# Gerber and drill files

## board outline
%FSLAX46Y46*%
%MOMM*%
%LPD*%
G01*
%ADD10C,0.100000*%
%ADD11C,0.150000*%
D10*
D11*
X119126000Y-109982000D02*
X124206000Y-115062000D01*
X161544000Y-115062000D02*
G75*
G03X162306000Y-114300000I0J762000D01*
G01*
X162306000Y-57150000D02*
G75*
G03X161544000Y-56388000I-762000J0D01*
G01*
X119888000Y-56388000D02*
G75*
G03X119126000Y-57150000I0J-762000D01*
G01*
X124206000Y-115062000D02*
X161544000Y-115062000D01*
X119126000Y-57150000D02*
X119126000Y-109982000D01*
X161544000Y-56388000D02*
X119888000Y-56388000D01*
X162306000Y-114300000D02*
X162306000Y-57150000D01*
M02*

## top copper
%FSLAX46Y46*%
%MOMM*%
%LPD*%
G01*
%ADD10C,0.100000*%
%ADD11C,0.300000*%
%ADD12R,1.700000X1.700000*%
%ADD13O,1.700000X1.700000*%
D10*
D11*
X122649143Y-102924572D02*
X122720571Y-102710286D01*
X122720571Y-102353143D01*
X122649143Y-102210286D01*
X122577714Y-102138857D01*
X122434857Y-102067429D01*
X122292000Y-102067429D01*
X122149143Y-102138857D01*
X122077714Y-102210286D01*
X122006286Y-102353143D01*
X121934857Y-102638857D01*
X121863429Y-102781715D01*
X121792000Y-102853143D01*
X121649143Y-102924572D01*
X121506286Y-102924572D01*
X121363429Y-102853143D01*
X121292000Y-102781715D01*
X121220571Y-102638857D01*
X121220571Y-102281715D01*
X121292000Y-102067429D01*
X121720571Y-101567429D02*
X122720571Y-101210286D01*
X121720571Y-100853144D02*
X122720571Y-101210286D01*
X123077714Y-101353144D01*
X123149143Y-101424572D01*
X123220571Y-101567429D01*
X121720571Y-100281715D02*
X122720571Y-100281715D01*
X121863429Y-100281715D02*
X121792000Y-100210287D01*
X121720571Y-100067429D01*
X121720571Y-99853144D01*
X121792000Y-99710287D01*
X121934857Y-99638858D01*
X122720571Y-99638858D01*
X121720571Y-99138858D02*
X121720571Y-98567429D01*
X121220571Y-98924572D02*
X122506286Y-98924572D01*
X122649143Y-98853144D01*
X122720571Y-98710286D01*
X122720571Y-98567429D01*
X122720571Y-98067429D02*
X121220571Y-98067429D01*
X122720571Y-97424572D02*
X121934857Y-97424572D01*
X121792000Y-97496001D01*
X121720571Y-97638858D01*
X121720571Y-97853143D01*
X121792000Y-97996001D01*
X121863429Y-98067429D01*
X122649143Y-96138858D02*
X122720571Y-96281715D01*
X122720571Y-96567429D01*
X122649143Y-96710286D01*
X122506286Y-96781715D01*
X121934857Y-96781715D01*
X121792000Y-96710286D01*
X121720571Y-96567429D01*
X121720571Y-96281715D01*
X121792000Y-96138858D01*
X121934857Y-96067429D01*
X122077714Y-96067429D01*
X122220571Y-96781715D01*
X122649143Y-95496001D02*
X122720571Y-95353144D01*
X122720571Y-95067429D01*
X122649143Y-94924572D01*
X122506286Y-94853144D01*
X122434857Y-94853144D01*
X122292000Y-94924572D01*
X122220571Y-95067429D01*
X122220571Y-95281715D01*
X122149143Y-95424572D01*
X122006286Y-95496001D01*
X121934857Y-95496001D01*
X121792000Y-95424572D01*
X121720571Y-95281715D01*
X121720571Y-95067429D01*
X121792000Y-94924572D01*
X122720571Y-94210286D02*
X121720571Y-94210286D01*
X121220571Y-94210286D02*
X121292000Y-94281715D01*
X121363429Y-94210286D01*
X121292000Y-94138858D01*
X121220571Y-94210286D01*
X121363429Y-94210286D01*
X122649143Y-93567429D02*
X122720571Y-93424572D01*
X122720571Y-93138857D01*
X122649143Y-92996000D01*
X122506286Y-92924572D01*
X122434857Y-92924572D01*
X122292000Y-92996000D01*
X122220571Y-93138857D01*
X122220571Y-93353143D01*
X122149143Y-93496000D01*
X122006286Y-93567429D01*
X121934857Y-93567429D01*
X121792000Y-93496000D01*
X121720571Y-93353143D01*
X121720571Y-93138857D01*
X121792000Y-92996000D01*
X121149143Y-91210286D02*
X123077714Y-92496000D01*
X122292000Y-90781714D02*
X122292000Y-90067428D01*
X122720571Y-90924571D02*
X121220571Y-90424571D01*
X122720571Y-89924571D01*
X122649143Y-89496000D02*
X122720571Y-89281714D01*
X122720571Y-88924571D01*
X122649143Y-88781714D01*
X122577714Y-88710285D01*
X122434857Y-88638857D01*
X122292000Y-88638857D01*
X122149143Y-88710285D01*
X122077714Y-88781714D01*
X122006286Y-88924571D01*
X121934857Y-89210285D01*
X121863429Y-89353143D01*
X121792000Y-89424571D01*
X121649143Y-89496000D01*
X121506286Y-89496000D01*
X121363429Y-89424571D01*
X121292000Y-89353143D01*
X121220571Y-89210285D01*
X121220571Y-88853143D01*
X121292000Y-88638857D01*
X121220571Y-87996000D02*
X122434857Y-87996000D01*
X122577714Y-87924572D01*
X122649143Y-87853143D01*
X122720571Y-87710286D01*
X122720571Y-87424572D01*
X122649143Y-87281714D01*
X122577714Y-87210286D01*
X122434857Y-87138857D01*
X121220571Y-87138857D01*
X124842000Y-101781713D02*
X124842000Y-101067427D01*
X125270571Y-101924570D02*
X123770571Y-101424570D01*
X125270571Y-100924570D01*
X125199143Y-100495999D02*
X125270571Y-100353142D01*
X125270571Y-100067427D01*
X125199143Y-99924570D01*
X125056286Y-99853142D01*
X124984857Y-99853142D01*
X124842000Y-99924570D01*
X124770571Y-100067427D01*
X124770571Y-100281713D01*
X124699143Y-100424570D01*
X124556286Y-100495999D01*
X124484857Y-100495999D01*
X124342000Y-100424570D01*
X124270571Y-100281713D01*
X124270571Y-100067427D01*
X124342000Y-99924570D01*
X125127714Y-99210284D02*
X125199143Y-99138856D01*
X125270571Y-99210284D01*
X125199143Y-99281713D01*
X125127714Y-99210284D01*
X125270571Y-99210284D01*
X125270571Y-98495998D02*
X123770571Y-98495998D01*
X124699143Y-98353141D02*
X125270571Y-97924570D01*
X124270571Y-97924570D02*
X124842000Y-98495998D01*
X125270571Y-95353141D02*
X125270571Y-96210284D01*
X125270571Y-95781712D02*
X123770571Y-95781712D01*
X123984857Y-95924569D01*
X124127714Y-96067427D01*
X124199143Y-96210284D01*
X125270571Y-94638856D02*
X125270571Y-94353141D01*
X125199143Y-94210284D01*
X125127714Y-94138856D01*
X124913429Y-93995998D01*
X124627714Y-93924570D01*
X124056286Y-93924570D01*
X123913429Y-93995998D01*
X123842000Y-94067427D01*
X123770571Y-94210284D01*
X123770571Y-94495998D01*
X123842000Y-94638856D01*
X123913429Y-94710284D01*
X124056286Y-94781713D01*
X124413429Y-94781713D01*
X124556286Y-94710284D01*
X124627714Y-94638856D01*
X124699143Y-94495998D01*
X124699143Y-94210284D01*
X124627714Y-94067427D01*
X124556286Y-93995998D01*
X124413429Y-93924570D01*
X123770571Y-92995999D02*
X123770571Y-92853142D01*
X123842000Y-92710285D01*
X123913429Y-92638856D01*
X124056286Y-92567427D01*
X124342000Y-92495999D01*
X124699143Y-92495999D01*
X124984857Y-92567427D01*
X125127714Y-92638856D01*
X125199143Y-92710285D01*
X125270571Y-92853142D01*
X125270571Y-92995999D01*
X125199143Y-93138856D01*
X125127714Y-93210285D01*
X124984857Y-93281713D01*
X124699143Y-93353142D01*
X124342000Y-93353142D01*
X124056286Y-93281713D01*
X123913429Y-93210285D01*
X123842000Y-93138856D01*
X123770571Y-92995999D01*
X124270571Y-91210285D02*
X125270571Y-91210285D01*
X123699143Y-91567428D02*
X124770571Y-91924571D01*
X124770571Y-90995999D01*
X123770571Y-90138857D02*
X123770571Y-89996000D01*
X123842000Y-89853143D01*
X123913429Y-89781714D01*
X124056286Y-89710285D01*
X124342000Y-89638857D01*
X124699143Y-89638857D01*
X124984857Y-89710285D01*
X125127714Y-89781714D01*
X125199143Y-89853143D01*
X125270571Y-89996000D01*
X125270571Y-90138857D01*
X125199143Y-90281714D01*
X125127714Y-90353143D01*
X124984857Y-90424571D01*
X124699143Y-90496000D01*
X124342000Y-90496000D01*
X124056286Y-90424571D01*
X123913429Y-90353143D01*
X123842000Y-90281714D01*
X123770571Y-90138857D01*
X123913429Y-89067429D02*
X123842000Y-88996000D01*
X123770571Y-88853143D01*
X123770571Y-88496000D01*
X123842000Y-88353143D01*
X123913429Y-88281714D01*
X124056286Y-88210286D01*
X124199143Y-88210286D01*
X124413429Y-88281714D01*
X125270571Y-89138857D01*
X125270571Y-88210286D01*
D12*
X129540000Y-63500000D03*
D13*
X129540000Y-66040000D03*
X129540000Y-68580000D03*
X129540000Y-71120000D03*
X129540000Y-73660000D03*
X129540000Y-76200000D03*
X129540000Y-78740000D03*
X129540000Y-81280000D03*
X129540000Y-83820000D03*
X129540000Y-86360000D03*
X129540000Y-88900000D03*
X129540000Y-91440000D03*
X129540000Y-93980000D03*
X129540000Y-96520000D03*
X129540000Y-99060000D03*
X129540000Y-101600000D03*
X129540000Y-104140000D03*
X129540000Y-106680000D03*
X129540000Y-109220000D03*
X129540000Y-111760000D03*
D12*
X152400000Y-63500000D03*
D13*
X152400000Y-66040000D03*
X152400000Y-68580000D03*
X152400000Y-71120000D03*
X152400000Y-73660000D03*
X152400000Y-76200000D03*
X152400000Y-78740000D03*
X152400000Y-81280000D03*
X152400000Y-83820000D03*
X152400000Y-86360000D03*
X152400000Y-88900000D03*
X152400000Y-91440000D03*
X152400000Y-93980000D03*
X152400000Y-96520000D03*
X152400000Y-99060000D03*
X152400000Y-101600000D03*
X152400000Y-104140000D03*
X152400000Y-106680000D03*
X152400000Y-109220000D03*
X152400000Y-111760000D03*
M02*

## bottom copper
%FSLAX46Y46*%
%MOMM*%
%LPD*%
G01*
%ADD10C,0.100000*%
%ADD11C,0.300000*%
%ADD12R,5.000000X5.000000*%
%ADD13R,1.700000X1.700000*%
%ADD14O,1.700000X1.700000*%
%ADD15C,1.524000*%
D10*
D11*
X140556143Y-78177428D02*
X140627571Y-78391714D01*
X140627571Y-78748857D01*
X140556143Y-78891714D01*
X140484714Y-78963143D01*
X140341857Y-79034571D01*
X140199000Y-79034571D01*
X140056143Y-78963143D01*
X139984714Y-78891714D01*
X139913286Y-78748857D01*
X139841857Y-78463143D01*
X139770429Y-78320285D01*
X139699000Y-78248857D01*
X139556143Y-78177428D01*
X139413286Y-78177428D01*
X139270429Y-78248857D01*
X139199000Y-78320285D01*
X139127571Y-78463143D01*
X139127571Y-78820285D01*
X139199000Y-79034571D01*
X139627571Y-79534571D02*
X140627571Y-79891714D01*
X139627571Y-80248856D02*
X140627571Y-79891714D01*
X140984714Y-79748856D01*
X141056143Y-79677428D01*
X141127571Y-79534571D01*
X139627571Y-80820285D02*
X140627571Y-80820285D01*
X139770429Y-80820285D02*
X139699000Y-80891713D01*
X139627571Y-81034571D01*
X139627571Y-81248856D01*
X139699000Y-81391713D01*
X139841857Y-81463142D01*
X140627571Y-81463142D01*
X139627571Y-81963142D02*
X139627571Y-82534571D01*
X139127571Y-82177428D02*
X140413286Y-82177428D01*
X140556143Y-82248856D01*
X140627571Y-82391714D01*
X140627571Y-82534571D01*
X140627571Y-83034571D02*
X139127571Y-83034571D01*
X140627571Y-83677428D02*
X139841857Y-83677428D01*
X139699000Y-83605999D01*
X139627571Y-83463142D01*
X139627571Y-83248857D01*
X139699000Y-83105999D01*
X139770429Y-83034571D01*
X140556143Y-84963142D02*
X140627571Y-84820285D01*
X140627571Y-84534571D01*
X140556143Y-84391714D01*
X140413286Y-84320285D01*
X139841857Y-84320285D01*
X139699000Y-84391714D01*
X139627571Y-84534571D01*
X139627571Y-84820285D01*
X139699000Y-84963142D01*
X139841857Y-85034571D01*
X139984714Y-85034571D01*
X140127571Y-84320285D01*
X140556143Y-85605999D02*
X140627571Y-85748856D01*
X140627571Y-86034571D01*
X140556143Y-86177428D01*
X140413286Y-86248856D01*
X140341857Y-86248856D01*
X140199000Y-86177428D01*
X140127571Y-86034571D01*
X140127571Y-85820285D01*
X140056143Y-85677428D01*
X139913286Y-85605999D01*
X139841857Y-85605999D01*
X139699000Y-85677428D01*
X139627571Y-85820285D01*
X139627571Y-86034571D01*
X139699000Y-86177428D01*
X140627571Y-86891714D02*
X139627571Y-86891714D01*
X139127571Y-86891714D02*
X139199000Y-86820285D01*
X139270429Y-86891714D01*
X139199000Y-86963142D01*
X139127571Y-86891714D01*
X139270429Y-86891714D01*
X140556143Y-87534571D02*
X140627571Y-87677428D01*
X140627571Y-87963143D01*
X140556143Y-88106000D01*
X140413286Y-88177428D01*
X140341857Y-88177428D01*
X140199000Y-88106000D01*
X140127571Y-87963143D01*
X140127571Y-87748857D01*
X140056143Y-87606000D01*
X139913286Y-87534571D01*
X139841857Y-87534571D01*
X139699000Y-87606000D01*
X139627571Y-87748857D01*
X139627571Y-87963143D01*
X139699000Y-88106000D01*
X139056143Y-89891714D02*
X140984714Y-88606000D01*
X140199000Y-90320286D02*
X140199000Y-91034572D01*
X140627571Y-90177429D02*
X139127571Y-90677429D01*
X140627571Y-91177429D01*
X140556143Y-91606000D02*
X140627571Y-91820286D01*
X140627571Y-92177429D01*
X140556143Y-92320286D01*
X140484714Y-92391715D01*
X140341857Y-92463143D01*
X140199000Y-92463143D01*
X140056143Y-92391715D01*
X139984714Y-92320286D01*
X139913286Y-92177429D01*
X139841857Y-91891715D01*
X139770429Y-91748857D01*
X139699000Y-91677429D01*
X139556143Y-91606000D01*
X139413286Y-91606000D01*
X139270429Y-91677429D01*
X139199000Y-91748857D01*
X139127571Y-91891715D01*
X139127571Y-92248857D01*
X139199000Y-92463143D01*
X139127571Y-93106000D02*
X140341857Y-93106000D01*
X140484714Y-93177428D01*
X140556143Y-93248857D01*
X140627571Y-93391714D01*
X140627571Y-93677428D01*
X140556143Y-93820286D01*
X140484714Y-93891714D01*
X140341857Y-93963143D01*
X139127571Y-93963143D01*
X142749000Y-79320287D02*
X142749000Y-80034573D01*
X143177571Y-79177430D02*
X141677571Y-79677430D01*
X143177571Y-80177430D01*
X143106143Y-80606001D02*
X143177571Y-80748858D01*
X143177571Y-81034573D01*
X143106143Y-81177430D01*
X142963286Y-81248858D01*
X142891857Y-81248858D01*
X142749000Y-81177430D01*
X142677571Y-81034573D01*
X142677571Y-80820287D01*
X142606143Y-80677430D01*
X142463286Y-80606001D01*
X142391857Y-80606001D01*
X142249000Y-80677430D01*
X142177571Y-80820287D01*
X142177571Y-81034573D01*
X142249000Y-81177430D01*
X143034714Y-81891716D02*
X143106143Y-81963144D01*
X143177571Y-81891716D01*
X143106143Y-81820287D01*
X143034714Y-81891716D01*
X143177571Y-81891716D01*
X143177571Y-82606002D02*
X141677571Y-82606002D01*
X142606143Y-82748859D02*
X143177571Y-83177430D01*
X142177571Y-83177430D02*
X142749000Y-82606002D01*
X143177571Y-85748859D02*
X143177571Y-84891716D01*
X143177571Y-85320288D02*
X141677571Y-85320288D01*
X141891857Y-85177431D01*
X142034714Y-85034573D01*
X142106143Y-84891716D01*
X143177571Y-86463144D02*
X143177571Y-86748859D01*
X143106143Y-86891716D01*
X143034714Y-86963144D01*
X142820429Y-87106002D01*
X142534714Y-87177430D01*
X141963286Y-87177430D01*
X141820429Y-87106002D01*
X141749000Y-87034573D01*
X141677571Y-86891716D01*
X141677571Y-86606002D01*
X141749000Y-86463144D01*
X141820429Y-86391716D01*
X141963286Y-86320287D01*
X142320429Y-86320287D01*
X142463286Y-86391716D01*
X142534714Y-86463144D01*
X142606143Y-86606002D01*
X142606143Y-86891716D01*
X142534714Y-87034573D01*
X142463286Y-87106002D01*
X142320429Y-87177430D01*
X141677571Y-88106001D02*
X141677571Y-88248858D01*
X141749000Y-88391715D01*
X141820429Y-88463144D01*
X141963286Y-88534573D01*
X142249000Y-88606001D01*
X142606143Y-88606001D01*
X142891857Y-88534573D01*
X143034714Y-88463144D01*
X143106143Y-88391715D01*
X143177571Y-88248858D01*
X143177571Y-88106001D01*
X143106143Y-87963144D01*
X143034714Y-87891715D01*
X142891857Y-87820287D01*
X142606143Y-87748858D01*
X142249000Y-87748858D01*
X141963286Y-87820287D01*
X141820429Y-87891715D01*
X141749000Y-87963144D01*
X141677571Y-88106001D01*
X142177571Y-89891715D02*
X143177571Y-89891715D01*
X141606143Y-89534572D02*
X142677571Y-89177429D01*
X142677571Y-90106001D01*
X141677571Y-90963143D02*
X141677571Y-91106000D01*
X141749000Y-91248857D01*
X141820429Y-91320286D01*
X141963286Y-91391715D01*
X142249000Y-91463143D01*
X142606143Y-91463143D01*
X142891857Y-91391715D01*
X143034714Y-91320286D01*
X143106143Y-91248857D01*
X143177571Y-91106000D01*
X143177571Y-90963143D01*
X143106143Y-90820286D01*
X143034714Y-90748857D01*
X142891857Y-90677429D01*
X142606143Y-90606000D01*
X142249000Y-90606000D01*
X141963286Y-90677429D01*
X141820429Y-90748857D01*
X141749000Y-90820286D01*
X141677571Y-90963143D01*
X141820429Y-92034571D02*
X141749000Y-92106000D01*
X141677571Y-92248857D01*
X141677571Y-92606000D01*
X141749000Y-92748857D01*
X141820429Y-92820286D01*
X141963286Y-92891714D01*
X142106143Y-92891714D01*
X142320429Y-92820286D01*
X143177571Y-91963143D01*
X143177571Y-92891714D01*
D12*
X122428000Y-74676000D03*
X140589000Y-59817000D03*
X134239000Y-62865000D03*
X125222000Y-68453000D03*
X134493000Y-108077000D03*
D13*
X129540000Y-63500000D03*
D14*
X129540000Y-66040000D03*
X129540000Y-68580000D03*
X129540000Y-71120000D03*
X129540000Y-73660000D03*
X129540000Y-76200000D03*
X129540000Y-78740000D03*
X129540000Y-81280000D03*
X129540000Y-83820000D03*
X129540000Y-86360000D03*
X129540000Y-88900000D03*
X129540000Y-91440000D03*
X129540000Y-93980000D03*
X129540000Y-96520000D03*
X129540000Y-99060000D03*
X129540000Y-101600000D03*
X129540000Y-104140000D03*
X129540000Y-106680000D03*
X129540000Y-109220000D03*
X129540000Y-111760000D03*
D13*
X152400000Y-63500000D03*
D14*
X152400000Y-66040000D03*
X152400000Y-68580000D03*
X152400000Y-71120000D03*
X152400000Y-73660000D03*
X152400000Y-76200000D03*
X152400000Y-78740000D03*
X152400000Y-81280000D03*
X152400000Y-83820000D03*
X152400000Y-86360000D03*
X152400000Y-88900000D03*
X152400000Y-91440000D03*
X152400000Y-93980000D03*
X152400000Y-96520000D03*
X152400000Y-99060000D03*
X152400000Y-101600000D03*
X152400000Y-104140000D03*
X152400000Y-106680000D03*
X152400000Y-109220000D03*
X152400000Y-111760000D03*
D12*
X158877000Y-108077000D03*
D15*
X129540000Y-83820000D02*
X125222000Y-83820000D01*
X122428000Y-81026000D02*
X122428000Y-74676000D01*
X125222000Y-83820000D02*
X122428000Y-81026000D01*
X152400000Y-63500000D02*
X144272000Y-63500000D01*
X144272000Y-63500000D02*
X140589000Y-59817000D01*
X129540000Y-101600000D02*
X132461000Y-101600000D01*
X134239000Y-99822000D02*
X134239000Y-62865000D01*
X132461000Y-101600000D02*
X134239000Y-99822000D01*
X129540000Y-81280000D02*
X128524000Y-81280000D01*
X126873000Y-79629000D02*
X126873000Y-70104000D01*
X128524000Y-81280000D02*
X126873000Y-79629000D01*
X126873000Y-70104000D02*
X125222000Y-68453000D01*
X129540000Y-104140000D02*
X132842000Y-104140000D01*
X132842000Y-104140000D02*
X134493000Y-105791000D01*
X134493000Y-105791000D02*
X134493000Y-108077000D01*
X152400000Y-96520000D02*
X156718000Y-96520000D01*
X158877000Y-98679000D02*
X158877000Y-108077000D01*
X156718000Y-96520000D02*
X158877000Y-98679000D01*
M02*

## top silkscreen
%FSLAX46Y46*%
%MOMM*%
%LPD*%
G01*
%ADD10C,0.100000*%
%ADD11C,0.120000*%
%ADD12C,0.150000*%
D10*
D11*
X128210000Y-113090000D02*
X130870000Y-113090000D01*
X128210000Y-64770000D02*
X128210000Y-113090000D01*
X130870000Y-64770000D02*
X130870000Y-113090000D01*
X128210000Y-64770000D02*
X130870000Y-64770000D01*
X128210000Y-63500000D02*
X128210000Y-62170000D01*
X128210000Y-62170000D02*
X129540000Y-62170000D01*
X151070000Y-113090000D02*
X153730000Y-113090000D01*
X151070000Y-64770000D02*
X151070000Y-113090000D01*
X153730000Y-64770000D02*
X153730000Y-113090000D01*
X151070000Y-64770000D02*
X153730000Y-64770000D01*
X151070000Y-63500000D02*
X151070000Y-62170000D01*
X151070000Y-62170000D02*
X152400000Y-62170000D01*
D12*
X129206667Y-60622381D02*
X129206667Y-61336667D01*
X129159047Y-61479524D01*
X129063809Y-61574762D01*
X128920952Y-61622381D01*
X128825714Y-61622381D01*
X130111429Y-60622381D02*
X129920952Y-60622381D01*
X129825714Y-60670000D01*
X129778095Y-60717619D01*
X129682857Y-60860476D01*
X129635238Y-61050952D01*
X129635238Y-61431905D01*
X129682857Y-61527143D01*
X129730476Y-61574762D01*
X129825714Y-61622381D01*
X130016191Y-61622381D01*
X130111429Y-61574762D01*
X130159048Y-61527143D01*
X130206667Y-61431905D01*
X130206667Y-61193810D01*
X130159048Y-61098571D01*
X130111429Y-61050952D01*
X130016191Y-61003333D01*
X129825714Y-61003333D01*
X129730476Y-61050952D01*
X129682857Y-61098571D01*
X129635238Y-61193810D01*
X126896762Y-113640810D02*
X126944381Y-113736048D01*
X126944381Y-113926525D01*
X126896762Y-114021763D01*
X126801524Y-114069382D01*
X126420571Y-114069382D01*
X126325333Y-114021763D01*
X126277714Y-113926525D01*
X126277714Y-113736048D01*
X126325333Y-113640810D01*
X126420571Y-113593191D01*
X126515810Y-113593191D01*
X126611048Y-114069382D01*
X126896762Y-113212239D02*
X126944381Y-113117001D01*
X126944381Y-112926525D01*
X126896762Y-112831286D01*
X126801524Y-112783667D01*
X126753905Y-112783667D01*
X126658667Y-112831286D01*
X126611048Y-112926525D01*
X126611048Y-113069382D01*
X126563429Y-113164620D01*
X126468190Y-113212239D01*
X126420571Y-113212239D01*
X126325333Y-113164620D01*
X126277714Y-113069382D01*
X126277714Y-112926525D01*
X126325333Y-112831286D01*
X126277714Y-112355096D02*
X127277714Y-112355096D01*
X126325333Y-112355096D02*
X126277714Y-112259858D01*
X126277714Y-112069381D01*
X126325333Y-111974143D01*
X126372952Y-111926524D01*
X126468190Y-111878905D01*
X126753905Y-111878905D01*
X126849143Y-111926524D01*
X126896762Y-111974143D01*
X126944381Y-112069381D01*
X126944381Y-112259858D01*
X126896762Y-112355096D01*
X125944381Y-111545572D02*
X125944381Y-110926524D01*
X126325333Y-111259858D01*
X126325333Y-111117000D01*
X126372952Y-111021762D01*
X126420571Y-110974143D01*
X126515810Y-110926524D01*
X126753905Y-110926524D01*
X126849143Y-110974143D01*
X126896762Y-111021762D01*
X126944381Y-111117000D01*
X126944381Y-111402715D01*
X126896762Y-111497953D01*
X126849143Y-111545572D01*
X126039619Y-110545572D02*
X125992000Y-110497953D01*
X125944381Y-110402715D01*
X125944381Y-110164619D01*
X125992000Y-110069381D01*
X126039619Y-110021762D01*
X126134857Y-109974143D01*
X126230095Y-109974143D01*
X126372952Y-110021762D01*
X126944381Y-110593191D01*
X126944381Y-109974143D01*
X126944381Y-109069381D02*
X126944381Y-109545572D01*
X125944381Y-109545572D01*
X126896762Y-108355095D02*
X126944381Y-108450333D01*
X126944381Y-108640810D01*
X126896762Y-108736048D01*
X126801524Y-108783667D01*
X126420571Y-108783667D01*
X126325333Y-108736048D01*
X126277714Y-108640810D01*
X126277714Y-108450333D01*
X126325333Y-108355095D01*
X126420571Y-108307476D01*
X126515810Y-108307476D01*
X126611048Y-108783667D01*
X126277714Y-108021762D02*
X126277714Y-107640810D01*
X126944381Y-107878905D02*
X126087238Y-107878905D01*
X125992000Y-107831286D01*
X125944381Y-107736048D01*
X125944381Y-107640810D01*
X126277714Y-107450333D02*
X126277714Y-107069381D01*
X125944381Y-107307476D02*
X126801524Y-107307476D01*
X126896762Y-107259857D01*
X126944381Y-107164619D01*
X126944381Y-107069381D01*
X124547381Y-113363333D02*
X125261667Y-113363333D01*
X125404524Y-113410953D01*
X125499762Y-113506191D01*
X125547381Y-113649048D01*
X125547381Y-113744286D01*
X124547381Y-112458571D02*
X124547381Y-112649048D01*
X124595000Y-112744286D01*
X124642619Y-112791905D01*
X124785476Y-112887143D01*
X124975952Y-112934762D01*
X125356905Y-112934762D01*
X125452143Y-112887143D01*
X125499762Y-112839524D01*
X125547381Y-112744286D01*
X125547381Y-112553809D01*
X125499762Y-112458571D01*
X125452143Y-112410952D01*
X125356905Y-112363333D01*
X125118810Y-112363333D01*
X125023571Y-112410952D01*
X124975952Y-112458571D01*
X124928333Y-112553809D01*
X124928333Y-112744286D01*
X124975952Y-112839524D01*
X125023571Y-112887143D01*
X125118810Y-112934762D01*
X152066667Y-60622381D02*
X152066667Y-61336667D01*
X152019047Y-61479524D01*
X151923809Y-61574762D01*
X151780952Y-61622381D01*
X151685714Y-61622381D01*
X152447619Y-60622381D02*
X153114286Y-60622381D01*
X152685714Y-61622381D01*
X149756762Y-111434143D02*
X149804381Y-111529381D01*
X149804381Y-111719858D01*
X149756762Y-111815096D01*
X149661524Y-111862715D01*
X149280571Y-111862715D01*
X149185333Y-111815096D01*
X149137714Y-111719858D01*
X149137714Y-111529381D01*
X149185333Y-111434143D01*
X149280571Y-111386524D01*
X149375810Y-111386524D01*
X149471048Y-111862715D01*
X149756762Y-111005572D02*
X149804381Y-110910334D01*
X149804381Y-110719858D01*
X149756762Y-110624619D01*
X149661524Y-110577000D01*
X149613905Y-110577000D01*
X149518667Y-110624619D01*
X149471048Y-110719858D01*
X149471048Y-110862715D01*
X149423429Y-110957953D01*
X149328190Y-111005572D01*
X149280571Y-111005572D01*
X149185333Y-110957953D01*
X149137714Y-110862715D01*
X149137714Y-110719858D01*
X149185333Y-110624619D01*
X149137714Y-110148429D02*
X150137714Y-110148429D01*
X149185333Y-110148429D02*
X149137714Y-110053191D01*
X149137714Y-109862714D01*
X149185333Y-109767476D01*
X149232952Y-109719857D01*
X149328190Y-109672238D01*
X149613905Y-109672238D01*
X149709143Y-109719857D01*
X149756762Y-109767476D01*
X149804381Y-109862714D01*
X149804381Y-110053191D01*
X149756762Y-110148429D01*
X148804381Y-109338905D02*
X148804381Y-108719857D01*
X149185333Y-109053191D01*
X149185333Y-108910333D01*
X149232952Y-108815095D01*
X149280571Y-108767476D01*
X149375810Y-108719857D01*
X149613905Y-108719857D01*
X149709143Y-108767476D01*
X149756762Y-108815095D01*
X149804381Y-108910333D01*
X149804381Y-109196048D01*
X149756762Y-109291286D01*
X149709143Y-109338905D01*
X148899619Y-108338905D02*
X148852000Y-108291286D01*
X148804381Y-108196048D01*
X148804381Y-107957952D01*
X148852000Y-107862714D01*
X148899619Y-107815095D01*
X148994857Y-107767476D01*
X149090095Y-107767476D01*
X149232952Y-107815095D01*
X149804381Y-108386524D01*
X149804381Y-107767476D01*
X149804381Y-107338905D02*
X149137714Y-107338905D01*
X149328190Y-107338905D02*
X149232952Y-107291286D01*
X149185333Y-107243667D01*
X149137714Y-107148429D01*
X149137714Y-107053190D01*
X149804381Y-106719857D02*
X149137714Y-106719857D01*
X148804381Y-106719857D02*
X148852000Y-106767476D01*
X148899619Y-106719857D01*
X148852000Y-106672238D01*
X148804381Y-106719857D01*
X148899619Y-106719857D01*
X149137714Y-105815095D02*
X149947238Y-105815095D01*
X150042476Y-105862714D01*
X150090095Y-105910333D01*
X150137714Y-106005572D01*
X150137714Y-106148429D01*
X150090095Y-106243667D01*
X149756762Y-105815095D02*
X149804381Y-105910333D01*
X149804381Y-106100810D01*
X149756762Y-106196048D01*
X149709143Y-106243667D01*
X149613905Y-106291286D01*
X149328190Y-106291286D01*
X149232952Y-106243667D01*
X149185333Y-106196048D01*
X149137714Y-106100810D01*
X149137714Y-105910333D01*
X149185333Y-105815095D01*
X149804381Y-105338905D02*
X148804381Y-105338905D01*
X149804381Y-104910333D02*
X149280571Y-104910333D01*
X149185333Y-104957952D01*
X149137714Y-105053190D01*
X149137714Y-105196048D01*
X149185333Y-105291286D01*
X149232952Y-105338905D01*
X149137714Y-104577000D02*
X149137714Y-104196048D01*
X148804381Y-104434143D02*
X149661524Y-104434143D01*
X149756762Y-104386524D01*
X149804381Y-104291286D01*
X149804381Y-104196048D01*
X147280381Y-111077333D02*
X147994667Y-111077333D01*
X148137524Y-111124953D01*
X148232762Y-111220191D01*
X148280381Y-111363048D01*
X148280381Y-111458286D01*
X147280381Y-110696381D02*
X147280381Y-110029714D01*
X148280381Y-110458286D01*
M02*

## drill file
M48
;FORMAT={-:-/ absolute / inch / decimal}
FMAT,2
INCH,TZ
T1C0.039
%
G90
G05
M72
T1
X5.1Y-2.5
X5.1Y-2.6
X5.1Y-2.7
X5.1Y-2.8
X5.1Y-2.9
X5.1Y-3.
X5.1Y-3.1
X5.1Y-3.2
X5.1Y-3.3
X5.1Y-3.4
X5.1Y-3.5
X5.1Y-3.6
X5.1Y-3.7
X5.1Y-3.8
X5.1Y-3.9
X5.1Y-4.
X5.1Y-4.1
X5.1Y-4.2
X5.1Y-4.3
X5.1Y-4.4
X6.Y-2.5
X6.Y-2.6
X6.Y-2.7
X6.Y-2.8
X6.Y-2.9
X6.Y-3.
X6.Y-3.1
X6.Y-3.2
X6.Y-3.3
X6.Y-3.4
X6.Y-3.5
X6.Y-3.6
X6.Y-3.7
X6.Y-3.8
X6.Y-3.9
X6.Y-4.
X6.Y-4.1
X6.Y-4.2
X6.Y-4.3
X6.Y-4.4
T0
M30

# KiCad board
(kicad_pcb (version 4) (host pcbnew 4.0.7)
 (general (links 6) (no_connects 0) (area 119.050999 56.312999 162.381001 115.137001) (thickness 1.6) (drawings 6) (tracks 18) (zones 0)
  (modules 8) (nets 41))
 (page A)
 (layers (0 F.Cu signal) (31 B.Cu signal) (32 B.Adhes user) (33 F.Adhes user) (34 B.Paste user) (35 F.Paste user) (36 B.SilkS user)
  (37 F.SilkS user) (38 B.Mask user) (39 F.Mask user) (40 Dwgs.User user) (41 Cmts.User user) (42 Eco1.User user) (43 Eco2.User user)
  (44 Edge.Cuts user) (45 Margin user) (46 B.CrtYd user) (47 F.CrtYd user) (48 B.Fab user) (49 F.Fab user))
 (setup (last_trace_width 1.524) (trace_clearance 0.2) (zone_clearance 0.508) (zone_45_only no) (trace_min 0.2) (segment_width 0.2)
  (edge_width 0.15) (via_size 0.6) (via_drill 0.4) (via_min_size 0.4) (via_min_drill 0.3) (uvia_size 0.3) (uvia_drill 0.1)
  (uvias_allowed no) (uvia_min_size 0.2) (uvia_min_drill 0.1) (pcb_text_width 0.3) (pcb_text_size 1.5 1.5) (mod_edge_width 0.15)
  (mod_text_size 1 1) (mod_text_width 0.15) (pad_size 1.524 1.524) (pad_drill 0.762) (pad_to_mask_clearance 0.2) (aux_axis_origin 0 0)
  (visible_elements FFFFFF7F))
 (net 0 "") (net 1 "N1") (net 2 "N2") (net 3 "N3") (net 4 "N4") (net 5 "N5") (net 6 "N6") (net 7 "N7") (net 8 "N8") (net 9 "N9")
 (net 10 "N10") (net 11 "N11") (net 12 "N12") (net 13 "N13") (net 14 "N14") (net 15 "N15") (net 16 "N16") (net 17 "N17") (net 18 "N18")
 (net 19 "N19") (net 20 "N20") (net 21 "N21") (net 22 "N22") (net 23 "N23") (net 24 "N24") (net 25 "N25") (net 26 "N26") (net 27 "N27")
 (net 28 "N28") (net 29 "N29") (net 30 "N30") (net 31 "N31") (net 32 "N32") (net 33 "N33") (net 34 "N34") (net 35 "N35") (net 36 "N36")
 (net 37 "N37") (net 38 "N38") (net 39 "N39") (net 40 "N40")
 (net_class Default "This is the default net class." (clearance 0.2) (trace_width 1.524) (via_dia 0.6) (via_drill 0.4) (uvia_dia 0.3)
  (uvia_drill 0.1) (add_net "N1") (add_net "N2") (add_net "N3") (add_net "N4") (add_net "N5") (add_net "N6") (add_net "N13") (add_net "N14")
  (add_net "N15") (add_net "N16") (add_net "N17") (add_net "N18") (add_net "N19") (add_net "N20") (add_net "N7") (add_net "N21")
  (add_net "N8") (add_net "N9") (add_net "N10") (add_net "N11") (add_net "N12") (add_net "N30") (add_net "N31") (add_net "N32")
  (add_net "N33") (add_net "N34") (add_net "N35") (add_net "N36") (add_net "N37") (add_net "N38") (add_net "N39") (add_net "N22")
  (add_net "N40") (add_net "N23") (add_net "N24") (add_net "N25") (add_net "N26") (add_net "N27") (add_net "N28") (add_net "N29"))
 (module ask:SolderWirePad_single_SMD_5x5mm (layer B.Cu) (at 122.428 74.676)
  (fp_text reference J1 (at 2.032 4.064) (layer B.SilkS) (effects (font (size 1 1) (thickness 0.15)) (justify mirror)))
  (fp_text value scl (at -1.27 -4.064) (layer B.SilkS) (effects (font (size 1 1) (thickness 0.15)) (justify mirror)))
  (pad 1 smd rect (at 0 0) (size 5 5) (layers B.Cu B.Paste B.Mask) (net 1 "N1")))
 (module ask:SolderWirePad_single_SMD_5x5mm (layer B.Cu) (at 140.589 59.817)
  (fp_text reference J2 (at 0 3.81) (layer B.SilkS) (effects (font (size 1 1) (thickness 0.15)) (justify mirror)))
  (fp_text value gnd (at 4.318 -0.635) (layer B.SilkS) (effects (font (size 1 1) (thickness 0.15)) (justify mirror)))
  (pad 1 smd rect (at 0 0) (size 5 5) (layers B.Cu B.Paste B.Mask) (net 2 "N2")))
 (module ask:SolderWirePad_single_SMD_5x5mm (layer B.Cu) (at 134.239 62.865)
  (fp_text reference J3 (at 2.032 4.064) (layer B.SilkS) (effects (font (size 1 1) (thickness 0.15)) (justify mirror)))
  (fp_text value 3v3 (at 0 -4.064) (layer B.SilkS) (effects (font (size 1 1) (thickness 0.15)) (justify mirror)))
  (pad 1 smd rect (at 0 0) (size 5 5) (layers B.Cu B.Paste B.Mask) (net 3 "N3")))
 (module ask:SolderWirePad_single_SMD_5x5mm (layer B.Cu) (at 125.222 68.453)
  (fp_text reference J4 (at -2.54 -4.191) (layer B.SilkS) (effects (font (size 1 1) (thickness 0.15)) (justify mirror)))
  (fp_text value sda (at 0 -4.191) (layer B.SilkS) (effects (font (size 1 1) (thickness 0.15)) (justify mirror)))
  (pad 1 smd rect (at 0 0) (size 5 5) (layers B.Cu B.Paste B.Mask) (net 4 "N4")))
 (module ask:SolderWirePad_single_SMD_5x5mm (layer B.Cu) (at 134.493 108.077)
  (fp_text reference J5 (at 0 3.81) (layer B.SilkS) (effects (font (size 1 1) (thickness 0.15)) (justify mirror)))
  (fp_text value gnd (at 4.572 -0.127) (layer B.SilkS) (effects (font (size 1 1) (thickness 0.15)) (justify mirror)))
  (pad 1 smd rect (at 0 0) (size 5 5) (layers B.Cu B.Paste B.Mask) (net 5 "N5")))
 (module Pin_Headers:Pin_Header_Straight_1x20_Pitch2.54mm (layer F.Cu) (at 129.54 63.5)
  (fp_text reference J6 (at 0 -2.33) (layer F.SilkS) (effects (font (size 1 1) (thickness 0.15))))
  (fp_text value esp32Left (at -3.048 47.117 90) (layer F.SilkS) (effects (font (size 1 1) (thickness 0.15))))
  (fp_line (start -1.33 49.59) (end 1.33 49.59) (layer F.SilkS) (width 0.12))
  (fp_line (start -1.33 1.27) (end -1.33 49.59) (layer F.SilkS) (width 0.12))
  (fp_line (start 1.33 1.27) (end 1.33 49.59) (layer F.SilkS) (width 0.12))
  (fp_line (start -1.33 1.27) (end 1.33 1.27) (layer F.SilkS) (width 0.12))
  (fp_line (start -1.33 0) (end -1.33 -1.33) (layer F.SilkS) (width 0.12))
  (fp_line (start -1.33 -1.33) (end 0 -1.33) (layer F.SilkS) (width 0.12))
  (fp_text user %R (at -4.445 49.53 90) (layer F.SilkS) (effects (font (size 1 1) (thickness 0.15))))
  (pad 1 thru_hole rect (at 0 0) (size 1.7 1.7) (drill 1) (layers *.Cu *.Mask) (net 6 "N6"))
  (pad 2 thru_hole oval (at 0 2.54) (size 1.7 1.7) (drill 1) (layers *.Cu *.Mask) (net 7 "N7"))
  (pad 3 thru_hole oval (at 0 5.08) (size 1.7 1.7) (drill 1) (layers *.Cu *.Mask) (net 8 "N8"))
  (pad 4 thru_hole oval (at 0 7.62) (size 1.7 1.7) (drill 1) (layers *.Cu *.Mask) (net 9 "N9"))
  (pad 5 thru_hole oval (at 0 10.16) (size 1.7 1.7) (drill 1) (layers *.Cu *.Mask) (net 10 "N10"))
  (pad 6 thru_hole oval (at 0 12.7) (size 1.7 1.7) (drill 1) (layers *.Cu *.Mask) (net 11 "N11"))
  (pad 7 thru_hole oval (at 0 15.24) (size 1.7 1.7) (drill 1) (layers *.Cu *.Mask) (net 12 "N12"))
  (pad 8 thru_hole oval (at 0 17.78) (size 1.7 1.7) (drill 1) (layers *.Cu *.Mask) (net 4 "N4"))
  (pad 9 thru_hole oval (at 0 20.32) (size 1.7 1.7) (drill 1) (layers *.Cu *.Mask) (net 1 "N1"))
  (pad 10 thru_hole oval (at 0 22.86) (size 1.7 1.7) (drill 1) (layers *.Cu *.Mask) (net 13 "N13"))
  (pad 11 thru_hole oval (at 0 25.4) (size 1.7 1.7) (drill 1) (layers *.Cu *.Mask) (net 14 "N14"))
  (pad 12 thru_hole oval (at 0 27.94) (size 1.7 1.7) (drill 1) (layers *.Cu *.Mask) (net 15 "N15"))
  (pad 13 thru_hole oval (at 0 30.48) (size 1.7 1.7) (drill 1) (layers *.Cu *.Mask) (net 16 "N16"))
  (pad 14 thru_hole oval (at 0 33.02) (size 1.7 1.7) (drill 1) (layers *.Cu *.Mask) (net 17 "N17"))
  (pad 15 thru_hole oval (at 0 35.56) (size 1.7 1.7) (drill 1) (layers *.Cu *.Mask) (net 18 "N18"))
  (pad 16 thru_hole oval (at 0 38.1) (size 1.7 1.7) (drill 1) (layers *.Cu *.Mask) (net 3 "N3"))
  (pad 17 thru_hole oval (at 0 40.64) (size 1.7 1.7) (drill 1) (layers *.Cu *.Mask) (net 5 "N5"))
  (pad 18 thru_hole oval (at 0 43.18) (size 1.7 1.7) (drill 1) (layers *.Cu *.Mask) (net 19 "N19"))
  (pad 19 thru_hole oval (at 0 45.72) (size 1.7 1.7) (drill 1) (layers *.Cu *.Mask) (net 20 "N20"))
  (pad 20 thru_hole oval (at 0 48.26) (size 1.7 1.7) (drill 1) (layers *.Cu *.Mask) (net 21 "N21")))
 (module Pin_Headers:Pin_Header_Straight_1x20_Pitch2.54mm (layer F.Cu) (at 152.4 63.5)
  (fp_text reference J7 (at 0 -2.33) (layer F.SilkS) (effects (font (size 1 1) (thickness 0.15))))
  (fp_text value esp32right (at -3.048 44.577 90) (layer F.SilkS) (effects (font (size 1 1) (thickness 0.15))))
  (fp_line (start -1.33 49.59) (end 1.33 49.59) (layer F.SilkS) (width 0.12))
  (fp_line (start -1.33 1.27) (end -1.33 49.59) (layer F.SilkS) (width 0.12))
  (fp_line (start 1.33 1.27) (end 1.33 49.59) (layer F.SilkS) (width 0.12))
  (fp_line (start -1.33 1.27) (end 1.33 1.27) (layer F.SilkS) (width 0.12))
  (fp_line (start -1.33 0) (end -1.33 -1.33) (layer F.SilkS) (width 0.12))
  (fp_line (start -1.33 -1.33) (end 0 -1.33) (layer F.SilkS) (width 0.12))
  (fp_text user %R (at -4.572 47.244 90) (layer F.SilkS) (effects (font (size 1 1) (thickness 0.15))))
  (pad 1 thru_hole rect (at 0 0) (size 1.7 1.7) (drill 1) (layers *.Cu *.Mask) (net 2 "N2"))
  (pad 2 thru_hole oval (at 0 2.54) (size 1.7 1.7) (drill 1) (layers *.Cu *.Mask) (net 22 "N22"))
  (pad 3 thru_hole oval (at 0 5.08) (size 1.7 1.7) (drill 1) (layers *.Cu *.Mask) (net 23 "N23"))
  (pad 4 thru_hole oval (at 0 7.62) (size 1.7 1.7) (drill 1) (layers *.Cu *.Mask) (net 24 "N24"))
  (pad 5 thru_hole oval (at 0 10.16) (size 1.7 1.7) (drill 1) (layers *.Cu *.Mask) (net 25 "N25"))
  (pad 6 thru_hole oval (at 0 12.7) (size 1.7 1.7) (drill 1) (layers *.Cu *.Mask) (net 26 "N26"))
  (pad 7 thru_hole oval (at 0 15.24) (size 1.7 1.7) (drill 1) (layers *.Cu *.Mask) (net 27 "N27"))
  (pad 8 thru_hole oval (at 0 17.78) (size 1.7 1.7) (drill 1) (layers *.Cu *.Mask) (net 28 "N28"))
  (pad 9 thru_hole oval (at 0 20.32) (size 1.7 1.7) (drill 1) (layers *.Cu *.Mask) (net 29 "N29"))
  (pad 10 thru_hole oval (at 0 22.86) (size 1.7 1.7) (drill 1) (layers *.Cu *.Mask) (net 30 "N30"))
  (pad 11 thru_hole oval (at 0 25.4) (size 1.7 1.7) (drill 1) (layers *.Cu *.Mask) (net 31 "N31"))
  (pad 12 thru_hole oval (at 0 27.94) (size 1.7 1.7) (drill 1) (layers *.Cu *.Mask) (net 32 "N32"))
  (pad 13 thru_hole oval (at 0 30.48) (size 1.7 1.7) (drill 1) (layers *.Cu *.Mask) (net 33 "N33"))
  (pad 14 thru_hole oval (at 0 33.02) (size 1.7 1.7) (drill 1) (layers *.Cu *.Mask) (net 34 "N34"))
  (pad 15 thru_hole oval (at 0 35.56) (size 1.7 1.7) (drill 1) (layers *.Cu *.Mask) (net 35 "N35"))
  (pad 16 thru_hole oval (at 0 38.1) (size 1.7 1.7) (drill 1) (layers *.Cu *.Mask) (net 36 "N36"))
  (pad 17 thru_hole oval (at 0 40.64) (size 1.7 1.7) (drill 1) (layers *.Cu *.Mask) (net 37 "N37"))
  (pad 18 thru_hole oval (at 0 43.18) (size 1.7 1.7) (drill 1) (layers *.Cu *.Mask) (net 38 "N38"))
  (pad 19 thru_hole oval (at 0 45.72) (size 1.7 1.7) (drill 1) (layers *.Cu *.Mask) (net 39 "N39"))
  (pad 20 thru_hole oval (at 0 48.26) (size 1.7 1.7) (drill 1) (layers *.Cu *.Mask) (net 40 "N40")))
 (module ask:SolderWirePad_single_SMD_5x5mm (layer B.Cu) (at 158.877 108.077)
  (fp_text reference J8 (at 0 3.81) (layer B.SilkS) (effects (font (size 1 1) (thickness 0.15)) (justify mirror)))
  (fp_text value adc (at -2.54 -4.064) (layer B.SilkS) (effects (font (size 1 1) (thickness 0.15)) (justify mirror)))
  (pad 1 smd rect (at 0 0) (size 5 5) (layers B.Cu B.Paste B.Mask) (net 34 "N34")))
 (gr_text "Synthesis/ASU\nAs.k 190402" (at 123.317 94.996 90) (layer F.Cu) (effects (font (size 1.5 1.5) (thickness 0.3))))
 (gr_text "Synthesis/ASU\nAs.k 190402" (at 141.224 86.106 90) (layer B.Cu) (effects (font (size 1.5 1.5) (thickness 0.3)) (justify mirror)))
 (gr_line (start 119.126 115.062) (end 162.306 115.062) (angle 90) (layer Edge.Cuts) (width 0.15))
 (gr_line (start 119.126 56.388) (end 119.126 115.062) (angle 90) (layer Edge.Cuts) (width 0.15))
 (gr_line (start 162.306 56.388) (end 119.126 56.388) (angle 90) (layer Edge.Cuts) (width 0.15))
 (gr_line (start 162.306 115.062) (end 162.306 56.388) (angle 90) (layer Edge.Cuts) (width 0.15))
 (segment (start 129.54 83.82) (end 125.222 83.82) (width 1.524) (layer B.Cu) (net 1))
 (segment (start 122.428 81.026) (end 122.428 74.676) (width 1.524) (layer B.Cu) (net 1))
 (segment (start 125.222 83.82) (end 122.428 81.026) (width 1.524) (layer B.Cu) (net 1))
 (segment (start 152.4 63.5) (end 144.272 63.5) (width 1.524) (layer B.Cu) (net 2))
 (segment (start 144.272 63.5) (end 140.589 59.817) (width 1.524) (layer B.Cu) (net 2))
 (segment (start 129.54 101.6) (end 132.461 101.6) (width 1.524) (layer B.Cu) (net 3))
 (segment (start 134.239 99.822) (end 134.239 62.865) (width 1.524) (layer B.Cu) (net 3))
 (segment (start 132.461 101.6) (end 134.239 99.822) (width 1.524) (layer B.Cu) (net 3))
 (segment (start 129.54 81.28) (end 128.524 81.28) (width 1.524) (layer B.Cu) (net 4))
 (segment (start 126.873 79.629) (end 126.873 70.104) (width 1.524) (layer B.Cu) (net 4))
 (segment (start 128.524 81.28) (end 126.873 79.629) (width 1.524) (layer B.Cu) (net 4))
 (segment (start 126.873 70.104) (end 125.222 68.453) (width 1.524) (layer B.Cu) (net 4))
 (segment (start 129.54 104.14) (end 132.842 104.14) (width 1.524) (layer B.Cu) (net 5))
 (segment (start 132.842 104.14) (end 134.493 105.791) (width 1.524) (layer B.Cu) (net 5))
 (segment (start 134.493 105.791) (end 134.493 108.077) (width 1.524) (layer B.Cu) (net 5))
 (segment (start 152.4 96.52) (end 156.718 96.52) (width 1.524) (layer B.Cu) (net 34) (status 400000))
 (segment (start 158.877 98.679) (end 158.877 108.077) (width 1.524) (layer B.Cu) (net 34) (status 800000))
 (segment (start 156.718 96.52) (end 158.877 98.679) (width 1.524) (layer B.Cu) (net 34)))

